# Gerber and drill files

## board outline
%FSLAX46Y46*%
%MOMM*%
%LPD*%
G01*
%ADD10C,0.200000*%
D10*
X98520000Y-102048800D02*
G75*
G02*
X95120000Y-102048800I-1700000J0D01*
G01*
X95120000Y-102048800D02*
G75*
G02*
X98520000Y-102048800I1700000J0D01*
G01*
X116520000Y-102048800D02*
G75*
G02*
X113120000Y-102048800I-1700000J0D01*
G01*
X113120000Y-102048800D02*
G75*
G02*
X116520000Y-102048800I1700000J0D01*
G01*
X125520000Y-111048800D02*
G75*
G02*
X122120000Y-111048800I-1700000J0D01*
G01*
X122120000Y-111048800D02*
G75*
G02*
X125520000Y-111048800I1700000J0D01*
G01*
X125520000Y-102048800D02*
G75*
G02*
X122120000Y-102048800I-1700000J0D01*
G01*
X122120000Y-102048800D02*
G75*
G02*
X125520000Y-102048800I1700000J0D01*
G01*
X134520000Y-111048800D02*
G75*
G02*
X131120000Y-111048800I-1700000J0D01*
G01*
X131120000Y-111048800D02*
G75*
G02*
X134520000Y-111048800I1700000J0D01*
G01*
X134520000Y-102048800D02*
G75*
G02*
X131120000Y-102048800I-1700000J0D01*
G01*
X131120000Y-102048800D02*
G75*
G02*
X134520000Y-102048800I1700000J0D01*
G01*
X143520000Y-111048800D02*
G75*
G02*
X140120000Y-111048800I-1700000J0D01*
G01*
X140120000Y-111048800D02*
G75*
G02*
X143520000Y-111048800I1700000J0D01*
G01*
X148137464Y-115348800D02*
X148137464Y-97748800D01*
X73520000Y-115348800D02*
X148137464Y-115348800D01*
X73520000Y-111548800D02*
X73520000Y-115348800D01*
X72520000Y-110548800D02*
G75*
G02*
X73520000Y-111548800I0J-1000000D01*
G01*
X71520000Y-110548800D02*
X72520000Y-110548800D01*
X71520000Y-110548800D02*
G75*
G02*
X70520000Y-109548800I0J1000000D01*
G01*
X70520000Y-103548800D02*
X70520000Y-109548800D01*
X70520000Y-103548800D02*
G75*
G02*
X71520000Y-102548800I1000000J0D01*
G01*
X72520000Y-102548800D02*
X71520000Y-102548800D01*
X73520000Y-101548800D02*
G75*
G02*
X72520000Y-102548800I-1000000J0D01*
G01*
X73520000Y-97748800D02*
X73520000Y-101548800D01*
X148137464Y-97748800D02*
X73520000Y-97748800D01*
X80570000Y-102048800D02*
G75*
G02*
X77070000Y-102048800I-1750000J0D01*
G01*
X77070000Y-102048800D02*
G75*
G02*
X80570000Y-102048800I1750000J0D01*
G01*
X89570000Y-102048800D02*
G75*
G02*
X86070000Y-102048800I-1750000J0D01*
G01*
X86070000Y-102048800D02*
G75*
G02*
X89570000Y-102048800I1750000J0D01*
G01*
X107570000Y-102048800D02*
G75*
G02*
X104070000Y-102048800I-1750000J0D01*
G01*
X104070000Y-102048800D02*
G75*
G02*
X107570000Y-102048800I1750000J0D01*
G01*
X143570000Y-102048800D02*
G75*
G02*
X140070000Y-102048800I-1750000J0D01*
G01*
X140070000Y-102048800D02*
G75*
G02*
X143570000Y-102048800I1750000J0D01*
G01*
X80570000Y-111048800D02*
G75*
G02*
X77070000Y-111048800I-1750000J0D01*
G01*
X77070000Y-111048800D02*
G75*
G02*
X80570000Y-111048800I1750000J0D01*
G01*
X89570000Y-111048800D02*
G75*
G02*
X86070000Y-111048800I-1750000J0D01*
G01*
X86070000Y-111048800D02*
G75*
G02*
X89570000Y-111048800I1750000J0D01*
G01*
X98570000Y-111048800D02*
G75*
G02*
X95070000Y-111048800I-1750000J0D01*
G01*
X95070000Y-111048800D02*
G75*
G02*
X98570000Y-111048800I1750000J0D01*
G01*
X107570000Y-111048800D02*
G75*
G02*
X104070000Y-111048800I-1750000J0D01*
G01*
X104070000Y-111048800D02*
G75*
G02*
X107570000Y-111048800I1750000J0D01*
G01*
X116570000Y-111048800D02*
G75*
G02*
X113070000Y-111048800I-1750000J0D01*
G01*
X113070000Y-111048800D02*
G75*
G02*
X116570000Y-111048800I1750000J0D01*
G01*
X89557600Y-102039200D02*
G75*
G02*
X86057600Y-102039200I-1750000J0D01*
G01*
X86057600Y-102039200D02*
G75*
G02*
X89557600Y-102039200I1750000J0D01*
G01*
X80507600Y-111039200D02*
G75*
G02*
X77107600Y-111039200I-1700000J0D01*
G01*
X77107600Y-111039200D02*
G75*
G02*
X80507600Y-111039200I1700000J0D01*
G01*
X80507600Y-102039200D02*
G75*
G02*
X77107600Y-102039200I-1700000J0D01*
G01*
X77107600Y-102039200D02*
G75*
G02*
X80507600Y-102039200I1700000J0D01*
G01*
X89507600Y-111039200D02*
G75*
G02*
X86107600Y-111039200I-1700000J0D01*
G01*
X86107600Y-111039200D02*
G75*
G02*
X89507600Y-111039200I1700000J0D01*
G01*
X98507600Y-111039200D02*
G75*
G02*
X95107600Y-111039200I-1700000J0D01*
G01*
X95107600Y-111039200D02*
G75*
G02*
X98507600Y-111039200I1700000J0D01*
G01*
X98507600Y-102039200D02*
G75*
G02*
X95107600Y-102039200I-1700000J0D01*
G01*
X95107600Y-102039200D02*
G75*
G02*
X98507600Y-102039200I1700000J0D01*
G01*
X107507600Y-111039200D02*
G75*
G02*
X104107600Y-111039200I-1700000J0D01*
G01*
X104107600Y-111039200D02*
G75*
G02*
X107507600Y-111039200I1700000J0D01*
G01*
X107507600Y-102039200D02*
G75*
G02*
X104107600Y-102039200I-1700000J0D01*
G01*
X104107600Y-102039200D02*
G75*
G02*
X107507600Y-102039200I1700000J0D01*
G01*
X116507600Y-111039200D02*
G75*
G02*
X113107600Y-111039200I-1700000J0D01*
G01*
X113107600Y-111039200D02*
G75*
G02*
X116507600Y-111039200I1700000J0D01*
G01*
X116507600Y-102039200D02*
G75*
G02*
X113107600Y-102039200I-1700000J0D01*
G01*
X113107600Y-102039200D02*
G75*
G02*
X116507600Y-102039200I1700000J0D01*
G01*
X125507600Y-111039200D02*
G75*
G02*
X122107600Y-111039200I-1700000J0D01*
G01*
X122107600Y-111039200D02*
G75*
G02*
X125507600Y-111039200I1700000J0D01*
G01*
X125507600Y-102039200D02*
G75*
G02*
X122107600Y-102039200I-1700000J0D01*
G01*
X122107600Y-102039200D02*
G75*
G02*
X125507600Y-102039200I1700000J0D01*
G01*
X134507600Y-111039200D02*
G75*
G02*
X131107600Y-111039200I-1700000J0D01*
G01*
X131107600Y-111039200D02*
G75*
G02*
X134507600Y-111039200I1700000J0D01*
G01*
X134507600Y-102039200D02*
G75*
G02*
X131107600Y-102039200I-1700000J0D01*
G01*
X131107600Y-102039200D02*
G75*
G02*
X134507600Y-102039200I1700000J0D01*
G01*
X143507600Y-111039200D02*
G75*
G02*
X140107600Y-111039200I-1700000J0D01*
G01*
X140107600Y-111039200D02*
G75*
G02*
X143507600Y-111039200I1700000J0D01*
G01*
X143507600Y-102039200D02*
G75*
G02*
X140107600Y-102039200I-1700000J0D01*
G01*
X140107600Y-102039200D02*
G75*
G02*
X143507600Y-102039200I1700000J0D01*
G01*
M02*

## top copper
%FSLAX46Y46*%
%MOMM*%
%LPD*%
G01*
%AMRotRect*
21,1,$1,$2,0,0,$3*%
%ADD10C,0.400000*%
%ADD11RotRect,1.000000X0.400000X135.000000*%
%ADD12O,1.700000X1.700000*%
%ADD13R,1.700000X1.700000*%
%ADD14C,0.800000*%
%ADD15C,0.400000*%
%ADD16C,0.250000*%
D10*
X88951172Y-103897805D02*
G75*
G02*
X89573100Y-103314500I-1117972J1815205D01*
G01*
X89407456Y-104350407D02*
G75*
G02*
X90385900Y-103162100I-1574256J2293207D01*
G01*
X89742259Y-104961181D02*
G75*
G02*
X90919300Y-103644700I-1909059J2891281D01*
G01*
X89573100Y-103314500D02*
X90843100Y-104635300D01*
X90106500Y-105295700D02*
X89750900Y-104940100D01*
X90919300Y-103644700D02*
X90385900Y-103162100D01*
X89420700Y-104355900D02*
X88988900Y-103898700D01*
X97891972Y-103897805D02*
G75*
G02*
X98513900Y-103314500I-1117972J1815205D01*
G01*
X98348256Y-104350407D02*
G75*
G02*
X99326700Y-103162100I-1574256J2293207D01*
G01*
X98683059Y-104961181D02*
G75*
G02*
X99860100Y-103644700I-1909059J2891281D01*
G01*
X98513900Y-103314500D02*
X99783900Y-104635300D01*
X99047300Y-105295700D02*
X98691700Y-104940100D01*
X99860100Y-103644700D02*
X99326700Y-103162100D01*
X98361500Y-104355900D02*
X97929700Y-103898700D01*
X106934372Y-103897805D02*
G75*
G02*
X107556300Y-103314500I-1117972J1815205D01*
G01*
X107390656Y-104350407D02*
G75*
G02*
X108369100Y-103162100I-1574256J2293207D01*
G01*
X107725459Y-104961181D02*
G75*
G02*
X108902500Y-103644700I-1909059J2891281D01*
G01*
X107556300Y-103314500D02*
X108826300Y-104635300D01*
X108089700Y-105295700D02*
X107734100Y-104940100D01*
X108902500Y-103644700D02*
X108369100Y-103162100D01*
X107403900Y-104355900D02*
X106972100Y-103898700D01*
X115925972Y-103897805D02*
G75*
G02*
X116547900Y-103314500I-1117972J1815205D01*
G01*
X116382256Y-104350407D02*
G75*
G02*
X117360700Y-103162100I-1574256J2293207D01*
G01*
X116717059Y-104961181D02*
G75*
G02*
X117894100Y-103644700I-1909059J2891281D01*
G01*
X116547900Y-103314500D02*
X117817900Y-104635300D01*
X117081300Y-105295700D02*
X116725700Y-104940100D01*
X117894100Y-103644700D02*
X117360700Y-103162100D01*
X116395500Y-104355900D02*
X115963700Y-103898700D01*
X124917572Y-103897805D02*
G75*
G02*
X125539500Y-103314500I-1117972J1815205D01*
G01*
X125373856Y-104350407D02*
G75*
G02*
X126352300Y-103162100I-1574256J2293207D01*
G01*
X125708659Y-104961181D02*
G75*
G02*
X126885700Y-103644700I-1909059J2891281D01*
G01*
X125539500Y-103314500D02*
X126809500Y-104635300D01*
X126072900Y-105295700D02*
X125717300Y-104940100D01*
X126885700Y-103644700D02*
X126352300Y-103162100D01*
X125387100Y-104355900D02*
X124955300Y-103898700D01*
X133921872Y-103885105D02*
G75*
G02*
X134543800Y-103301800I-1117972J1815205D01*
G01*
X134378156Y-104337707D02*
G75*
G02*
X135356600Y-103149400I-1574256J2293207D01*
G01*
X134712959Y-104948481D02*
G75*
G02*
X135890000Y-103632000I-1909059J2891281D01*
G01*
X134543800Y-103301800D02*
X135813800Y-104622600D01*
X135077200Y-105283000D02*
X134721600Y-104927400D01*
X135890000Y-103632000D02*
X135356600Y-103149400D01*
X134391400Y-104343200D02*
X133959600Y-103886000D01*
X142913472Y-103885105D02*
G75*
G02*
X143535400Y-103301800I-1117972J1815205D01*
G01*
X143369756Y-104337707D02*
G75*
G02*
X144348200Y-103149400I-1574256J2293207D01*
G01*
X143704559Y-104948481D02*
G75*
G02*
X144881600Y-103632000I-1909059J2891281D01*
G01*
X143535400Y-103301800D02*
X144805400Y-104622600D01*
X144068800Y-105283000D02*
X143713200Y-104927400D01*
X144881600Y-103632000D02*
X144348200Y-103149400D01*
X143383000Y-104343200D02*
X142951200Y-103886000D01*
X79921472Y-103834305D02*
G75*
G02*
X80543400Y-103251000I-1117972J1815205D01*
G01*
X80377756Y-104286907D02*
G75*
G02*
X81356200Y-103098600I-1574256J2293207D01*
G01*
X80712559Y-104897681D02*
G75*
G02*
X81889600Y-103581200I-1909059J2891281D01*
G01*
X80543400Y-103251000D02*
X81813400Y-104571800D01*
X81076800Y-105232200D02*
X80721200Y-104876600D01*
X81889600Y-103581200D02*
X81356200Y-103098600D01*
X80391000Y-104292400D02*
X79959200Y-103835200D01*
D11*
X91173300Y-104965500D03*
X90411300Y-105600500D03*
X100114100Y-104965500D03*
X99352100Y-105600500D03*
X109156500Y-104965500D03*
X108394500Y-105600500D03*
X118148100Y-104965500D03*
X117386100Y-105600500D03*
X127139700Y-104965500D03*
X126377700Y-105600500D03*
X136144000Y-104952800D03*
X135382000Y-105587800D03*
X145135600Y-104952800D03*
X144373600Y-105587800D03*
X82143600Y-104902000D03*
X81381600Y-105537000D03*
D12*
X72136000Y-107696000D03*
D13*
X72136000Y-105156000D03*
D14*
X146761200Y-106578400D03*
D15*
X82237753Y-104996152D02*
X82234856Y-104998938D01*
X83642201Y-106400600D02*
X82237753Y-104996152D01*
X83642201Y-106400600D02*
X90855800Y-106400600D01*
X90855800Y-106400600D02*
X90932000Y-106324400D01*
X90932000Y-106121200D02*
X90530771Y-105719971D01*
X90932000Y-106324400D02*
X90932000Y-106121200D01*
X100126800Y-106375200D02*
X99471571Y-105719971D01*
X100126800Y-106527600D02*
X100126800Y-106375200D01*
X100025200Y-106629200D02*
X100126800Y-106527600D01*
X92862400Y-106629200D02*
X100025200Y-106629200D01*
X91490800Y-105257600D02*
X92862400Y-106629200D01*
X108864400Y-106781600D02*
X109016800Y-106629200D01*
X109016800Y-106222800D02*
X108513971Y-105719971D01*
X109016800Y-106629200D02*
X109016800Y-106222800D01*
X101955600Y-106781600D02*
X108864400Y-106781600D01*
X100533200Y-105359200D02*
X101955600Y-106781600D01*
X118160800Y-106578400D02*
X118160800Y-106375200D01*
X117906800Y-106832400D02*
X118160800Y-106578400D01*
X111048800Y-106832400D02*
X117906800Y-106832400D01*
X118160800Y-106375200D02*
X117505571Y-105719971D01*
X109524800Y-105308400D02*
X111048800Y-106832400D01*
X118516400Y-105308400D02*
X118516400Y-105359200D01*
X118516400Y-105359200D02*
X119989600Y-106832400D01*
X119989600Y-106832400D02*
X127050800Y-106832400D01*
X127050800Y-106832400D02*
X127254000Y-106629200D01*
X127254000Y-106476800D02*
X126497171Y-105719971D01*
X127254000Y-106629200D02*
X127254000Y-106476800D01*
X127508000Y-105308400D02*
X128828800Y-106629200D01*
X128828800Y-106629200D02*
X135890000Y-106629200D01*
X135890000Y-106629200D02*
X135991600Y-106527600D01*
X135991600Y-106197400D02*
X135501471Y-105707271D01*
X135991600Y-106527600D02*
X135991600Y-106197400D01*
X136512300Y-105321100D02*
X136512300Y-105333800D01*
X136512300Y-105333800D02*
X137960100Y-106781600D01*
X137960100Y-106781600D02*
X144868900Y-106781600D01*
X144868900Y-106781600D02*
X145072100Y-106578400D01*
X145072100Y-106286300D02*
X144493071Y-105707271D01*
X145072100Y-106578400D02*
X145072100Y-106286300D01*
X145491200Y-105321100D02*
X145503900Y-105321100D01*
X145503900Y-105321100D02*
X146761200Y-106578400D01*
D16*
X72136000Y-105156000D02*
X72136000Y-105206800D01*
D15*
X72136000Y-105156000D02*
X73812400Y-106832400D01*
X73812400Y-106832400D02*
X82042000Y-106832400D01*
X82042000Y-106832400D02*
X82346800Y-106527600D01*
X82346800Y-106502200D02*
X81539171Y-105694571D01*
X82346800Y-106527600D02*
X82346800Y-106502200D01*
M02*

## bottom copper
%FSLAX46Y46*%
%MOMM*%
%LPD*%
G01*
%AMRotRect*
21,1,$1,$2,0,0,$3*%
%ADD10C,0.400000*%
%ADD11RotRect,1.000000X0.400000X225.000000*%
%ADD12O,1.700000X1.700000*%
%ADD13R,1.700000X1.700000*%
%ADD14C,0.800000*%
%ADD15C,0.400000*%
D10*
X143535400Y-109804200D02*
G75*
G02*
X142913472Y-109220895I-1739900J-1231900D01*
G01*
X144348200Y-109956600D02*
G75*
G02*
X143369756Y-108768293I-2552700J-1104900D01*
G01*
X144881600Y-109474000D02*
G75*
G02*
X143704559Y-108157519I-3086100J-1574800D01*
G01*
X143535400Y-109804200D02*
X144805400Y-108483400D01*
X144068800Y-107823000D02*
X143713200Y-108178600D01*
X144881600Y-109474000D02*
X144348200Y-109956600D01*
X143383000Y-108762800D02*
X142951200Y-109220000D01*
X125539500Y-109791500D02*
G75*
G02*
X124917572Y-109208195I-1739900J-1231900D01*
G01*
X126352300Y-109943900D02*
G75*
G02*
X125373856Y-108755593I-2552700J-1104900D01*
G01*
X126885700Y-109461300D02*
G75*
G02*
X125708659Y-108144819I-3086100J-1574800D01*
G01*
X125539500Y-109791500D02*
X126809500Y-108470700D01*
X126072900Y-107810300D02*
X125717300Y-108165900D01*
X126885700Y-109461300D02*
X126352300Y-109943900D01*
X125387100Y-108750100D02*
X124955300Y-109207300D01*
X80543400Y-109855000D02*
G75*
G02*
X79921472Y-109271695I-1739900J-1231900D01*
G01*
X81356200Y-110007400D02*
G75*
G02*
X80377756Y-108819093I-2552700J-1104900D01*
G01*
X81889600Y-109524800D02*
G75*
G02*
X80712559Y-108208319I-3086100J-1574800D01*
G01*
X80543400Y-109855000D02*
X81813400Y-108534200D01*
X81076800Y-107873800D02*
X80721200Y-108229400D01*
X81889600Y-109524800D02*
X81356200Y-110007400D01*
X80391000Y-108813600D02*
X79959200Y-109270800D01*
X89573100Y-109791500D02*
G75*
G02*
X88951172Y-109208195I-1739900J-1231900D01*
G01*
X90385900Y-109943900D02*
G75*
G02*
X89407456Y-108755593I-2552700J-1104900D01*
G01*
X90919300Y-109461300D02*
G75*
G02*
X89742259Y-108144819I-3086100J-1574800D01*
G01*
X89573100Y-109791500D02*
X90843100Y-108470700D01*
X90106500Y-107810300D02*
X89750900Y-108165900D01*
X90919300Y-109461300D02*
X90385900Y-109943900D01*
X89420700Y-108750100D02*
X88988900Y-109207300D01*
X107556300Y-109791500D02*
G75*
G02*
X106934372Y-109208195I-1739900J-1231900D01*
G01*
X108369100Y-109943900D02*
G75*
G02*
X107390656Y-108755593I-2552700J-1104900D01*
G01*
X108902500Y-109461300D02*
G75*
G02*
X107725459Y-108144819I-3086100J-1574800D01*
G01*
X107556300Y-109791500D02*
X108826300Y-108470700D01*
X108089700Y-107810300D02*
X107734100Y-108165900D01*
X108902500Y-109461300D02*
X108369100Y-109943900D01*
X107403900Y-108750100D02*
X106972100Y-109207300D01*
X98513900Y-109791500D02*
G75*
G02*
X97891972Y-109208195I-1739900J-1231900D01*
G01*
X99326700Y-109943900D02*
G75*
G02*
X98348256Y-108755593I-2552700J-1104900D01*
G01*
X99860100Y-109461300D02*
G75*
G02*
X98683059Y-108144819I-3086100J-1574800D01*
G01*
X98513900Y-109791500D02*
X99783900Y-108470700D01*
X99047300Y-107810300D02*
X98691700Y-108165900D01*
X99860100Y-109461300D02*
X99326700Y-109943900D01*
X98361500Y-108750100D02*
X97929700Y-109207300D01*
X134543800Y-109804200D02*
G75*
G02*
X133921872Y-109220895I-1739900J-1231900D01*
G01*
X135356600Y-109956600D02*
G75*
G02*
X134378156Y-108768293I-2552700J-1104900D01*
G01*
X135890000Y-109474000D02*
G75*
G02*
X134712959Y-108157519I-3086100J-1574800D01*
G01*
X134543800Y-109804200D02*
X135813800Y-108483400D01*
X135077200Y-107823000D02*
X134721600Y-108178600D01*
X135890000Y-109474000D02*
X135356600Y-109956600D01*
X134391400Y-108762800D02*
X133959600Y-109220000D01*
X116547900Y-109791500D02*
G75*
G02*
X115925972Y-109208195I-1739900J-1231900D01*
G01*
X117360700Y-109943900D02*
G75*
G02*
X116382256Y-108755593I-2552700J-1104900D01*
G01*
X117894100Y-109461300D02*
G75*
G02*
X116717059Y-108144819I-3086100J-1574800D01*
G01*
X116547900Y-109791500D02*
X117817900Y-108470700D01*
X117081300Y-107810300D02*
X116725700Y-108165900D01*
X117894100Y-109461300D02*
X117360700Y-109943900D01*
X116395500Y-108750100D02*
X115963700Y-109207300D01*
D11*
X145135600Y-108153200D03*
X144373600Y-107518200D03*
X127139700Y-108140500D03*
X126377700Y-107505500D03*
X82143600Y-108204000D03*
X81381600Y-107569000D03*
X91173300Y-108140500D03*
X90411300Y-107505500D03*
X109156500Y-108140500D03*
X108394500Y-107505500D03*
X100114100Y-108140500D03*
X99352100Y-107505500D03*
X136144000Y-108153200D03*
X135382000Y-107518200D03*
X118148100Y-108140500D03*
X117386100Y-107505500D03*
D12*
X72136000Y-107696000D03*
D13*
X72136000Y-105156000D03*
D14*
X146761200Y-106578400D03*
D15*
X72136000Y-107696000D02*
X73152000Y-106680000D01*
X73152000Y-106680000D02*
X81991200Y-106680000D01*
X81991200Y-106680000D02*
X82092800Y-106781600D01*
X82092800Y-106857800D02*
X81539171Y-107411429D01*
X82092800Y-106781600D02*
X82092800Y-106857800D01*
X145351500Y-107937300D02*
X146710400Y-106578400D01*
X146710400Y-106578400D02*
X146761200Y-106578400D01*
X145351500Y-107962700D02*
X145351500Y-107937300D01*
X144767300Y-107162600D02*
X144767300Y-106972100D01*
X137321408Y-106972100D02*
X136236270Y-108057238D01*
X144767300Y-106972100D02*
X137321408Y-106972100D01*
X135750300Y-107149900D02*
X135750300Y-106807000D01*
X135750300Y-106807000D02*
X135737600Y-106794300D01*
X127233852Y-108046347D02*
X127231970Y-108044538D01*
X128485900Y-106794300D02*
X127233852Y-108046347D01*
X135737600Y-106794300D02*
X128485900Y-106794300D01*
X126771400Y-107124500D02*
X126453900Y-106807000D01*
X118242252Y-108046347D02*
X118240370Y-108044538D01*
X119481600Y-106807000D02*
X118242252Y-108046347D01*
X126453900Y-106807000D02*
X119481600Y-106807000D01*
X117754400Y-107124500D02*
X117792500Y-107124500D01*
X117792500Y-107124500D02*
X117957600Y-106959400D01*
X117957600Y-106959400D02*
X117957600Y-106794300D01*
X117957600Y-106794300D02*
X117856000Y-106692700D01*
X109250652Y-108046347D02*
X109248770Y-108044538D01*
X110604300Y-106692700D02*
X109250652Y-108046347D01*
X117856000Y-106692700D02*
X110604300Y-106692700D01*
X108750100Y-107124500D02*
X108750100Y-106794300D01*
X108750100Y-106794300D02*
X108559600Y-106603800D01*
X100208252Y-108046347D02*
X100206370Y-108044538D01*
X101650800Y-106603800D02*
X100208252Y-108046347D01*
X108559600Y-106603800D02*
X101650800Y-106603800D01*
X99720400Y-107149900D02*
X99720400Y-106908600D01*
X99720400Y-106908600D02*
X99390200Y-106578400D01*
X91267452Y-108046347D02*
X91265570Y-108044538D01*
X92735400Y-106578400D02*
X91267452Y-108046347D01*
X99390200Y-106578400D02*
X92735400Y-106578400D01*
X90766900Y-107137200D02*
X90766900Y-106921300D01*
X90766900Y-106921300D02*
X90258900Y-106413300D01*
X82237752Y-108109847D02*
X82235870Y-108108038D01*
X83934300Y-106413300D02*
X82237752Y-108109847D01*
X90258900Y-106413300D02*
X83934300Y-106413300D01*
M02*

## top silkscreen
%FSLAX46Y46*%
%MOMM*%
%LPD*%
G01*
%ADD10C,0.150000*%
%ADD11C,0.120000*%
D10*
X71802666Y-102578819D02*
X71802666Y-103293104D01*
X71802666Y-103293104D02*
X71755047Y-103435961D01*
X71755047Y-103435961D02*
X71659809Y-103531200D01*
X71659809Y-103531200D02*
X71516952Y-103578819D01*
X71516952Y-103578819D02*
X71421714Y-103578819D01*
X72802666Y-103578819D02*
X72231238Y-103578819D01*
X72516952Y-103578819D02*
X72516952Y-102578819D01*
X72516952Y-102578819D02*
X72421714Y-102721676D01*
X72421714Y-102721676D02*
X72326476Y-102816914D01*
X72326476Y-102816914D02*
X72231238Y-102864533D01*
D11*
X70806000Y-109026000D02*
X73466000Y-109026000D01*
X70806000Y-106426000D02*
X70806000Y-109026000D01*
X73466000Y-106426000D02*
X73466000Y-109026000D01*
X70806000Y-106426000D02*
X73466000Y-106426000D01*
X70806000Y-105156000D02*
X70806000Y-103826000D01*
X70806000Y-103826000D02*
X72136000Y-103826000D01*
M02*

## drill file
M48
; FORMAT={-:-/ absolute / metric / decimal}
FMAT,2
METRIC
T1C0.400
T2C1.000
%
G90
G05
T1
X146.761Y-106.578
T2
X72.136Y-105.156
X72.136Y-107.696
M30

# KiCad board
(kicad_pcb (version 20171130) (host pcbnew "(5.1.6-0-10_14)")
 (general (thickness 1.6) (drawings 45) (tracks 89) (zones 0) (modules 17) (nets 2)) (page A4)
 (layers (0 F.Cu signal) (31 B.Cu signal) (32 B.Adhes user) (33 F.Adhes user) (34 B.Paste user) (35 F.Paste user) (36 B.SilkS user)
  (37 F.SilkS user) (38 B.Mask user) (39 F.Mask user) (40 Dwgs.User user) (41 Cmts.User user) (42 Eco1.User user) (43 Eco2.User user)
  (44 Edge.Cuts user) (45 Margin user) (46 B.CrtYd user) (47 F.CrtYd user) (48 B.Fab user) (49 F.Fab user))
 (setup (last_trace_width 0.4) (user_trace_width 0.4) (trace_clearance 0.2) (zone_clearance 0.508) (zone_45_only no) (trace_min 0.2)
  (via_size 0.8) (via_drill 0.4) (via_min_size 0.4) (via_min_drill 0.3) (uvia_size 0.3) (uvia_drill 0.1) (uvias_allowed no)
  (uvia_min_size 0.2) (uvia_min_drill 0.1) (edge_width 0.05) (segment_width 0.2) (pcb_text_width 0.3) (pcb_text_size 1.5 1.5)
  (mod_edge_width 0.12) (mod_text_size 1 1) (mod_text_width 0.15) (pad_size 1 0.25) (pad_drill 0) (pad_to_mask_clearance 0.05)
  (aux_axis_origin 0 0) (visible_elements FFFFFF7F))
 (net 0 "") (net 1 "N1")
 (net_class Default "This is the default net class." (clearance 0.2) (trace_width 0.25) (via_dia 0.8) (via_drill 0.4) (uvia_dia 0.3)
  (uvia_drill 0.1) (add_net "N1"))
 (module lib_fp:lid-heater (layer F.Cu) (at 88.1761 108.2167)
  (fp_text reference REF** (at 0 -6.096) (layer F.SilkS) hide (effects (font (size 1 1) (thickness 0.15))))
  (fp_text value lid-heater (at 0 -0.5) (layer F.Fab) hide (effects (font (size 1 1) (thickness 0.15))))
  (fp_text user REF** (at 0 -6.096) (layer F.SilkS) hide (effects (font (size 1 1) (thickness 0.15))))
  (fp_arc (start -0.3429 -6.1341) (end 1.397 -4.9022) (angle -336.9282282) (layer F.Cu) (width 0.4))
  (fp_arc (start -0.3429 -6.1595) (end 2.2098 -5.0546) (angle -327.8737649) (layer F.Cu) (width 0.4))
  (fp_arc (start -0.3429 -6.1468) (end 2.7432 -4.572) (angle -330.4707161) (layer F.Cu) (width 0.4))
  (fp_line (start 1.397 -4.9022) (end 2.667 -3.5814) (layer F.Cu) (width 0.4))
  (fp_line (start 1.9304 -2.921) (end 1.5748 -3.2766) (layer F.Cu) (width 0.4))
  (fp_line (start 2.7432 -4.572) (end 2.2098 -5.0546) (layer F.Cu) (width 0.4))
  (fp_line (start 1.2446 -3.8608) (end 0.8128 -4.318) (layer F.Cu) (width 0.4))
  (pad 1 smd rect (at 2.9972 -3.2512 135) (size 1 0.4) (layers F.Cu F.Paste))
  (pad 1 smd rect (at 2.2352 -2.6162 135) (size 1 0.4) (layers F.Cu F.Paste)))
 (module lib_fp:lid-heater (layer F.Cu) (at 97.1169 108.2167)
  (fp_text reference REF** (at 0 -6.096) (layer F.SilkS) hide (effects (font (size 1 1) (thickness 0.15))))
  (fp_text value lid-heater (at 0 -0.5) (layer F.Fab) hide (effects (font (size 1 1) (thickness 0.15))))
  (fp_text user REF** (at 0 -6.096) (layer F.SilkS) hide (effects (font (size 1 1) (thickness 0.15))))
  (fp_arc (start -0.3429 -6.1341) (end 1.397 -4.9022) (angle -336.9282282) (layer F.Cu) (width 0.4))
  (fp_arc (start -0.3429 -6.1595) (end 2.2098 -5.0546) (angle -327.8737649) (layer F.Cu) (width 0.4))
  (fp_arc (start -0.3429 -6.1468) (end 2.7432 -4.572) (angle -330.4707161) (layer F.Cu) (width 0.4))
  (fp_line (start 1.397 -4.9022) (end 2.667 -3.5814) (layer F.Cu) (width 0.4))
  (fp_line (start 1.9304 -2.921) (end 1.5748 -3.2766) (layer F.Cu) (width 0.4))
  (fp_line (start 2.7432 -4.572) (end 2.2098 -5.0546) (layer F.Cu) (width 0.4))
  (fp_line (start 1.2446 -3.8608) (end 0.8128 -4.318) (layer F.Cu) (width 0.4))
  (pad 1 smd rect (at 2.9972 -3.2512 135) (size 1 0.4) (layers F.Cu F.Paste))
  (pad 1 smd rect (at 2.2352 -2.6162 135) (size 1 0.4) (layers F.Cu F.Paste)))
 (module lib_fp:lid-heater (layer F.Cu) (at 106.1593 108.2167)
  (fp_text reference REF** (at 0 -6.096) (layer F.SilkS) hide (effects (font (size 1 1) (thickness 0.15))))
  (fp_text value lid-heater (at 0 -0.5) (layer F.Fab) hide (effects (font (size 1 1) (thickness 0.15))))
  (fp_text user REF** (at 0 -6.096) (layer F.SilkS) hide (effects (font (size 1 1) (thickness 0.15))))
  (fp_arc (start -0.3429 -6.1341) (end 1.397 -4.9022) (angle -336.9282282) (layer F.Cu) (width 0.4))
  (fp_arc (start -0.3429 -6.1595) (end 2.2098 -5.0546) (angle -327.8737649) (layer F.Cu) (width 0.4))
  (fp_arc (start -0.3429 -6.1468) (end 2.7432 -4.572) (angle -330.4707161) (layer F.Cu) (width 0.4))
  (fp_line (start 1.397 -4.9022) (end 2.667 -3.5814) (layer F.Cu) (width 0.4))
  (fp_line (start 1.9304 -2.921) (end 1.5748 -3.2766) (layer F.Cu) (width 0.4))
  (fp_line (start 2.7432 -4.572) (end 2.2098 -5.0546) (layer F.Cu) (width 0.4))
  (fp_line (start 1.2446 -3.8608) (end 0.8128 -4.318) (layer F.Cu) (width 0.4))
  (pad 1 smd rect (at 2.9972 -3.2512 135) (size 1 0.4) (layers F.Cu F.Paste))
  (pad 1 smd rect (at 2.2352 -2.6162 135) (size 1 0.4) (layers F.Cu F.Paste)))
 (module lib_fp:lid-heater (layer F.Cu) (at 115.1509 108.2167)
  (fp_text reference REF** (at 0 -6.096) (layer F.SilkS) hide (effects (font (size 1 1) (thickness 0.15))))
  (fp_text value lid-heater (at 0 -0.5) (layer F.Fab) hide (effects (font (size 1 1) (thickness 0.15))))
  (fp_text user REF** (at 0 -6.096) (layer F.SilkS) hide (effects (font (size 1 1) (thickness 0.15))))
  (fp_arc (start -0.3429 -6.1341) (end 1.397 -4.9022) (angle -336.9282282) (layer F.Cu) (width 0.4))
  (fp_arc (start -0.3429 -6.1595) (end 2.2098 -5.0546) (angle -327.8737649) (layer F.Cu) (width 0.4))
  (fp_arc (start -0.3429 -6.1468) (end 2.7432 -4.572) (angle -330.4707161) (layer F.Cu) (width 0.4))
  (fp_line (start 1.397 -4.9022) (end 2.667 -3.5814) (layer F.Cu) (width 0.4))
  (fp_line (start 1.9304 -2.921) (end 1.5748 -3.2766) (layer F.Cu) (width 0.4))
  (fp_line (start 2.7432 -4.572) (end 2.2098 -5.0546) (layer F.Cu) (width 0.4))
  (fp_line (start 1.2446 -3.8608) (end 0.8128 -4.318) (layer F.Cu) (width 0.4))
  (pad 1 smd rect (at 2.9972 -3.2512 135) (size 1 0.4) (layers F.Cu F.Paste))
  (pad 1 smd rect (at 2.2352 -2.6162 135) (size 1 0.4) (layers F.Cu F.Paste)))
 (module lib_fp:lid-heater (layer F.Cu) (at 124.1425 108.2167)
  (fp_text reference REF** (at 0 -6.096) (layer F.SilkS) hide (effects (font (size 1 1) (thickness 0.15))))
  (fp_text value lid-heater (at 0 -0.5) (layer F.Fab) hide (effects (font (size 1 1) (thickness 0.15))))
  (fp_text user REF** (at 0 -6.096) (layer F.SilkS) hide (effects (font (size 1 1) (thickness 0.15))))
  (fp_arc (start -0.3429 -6.1341) (end 1.397 -4.9022) (angle -336.9282282) (layer F.Cu) (width 0.4))
  (fp_arc (start -0.3429 -6.1595) (end 2.2098 -5.0546) (angle -327.8737649) (layer F.Cu) (width 0.4))
  (fp_arc (start -0.3429 -6.1468) (end 2.7432 -4.572) (angle -330.4707161) (layer F.Cu) (width 0.4))
  (fp_line (start 1.397 -4.9022) (end 2.667 -3.5814) (layer F.Cu) (width 0.4))
  (fp_line (start 1.9304 -2.921) (end 1.5748 -3.2766) (layer F.Cu) (width 0.4))
  (fp_line (start 2.7432 -4.572) (end 2.2098 -5.0546) (layer F.Cu) (width 0.4))
  (fp_line (start 1.2446 -3.8608) (end 0.8128 -4.318) (layer F.Cu) (width 0.4))
  (pad 1 smd rect (at 2.9972 -3.2512 135) (size 1 0.4) (layers F.Cu F.Paste))
  (pad 1 smd rect (at 2.2352 -2.6162 135) (size 1 0.4) (layers F.Cu F.Paste)))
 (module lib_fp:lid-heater (layer F.Cu) (at 133.1468 108.204)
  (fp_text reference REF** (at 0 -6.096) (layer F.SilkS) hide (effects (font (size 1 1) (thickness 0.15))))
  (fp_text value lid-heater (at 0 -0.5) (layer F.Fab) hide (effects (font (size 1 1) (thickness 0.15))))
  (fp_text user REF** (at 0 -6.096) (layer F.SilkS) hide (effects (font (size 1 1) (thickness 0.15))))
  (fp_arc (start -0.3429 -6.1341) (end 1.397 -4.9022) (angle -336.9282282) (layer F.Cu) (width 0.4))
  (fp_arc (start -0.3429 -6.1595) (end 2.2098 -5.0546) (angle -327.8737649) (layer F.Cu) (width 0.4))
  (fp_arc (start -0.3429 -6.1468) (end 2.7432 -4.572) (angle -330.4707161) (layer F.Cu) (width 0.4))
  (fp_line (start 1.397 -4.9022) (end 2.667 -3.5814) (layer F.Cu) (width 0.4))
  (fp_line (start 1.9304 -2.921) (end 1.5748 -3.2766) (layer F.Cu) (width 0.4))
  (fp_line (start 2.7432 -4.572) (end 2.2098 -5.0546) (layer F.Cu) (width 0.4))
  (fp_line (start 1.2446 -3.8608) (end 0.8128 -4.318) (layer F.Cu) (width 0.4))
  (pad 1 smd rect (at 2.9972 -3.2512 135) (size 1 0.4) (layers F.Cu F.Paste))
  (pad 1 smd rect (at 2.2352 -2.6162 135) (size 1 0.4) (layers F.Cu F.Paste)))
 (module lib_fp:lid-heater (layer F.Cu) (at 142.1384 108.204)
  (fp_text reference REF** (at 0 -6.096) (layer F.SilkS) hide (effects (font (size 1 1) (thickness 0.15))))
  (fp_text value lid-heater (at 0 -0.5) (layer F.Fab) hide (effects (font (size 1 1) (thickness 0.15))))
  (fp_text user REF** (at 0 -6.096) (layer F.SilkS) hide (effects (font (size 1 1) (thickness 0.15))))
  (fp_arc (start -0.3429 -6.1341) (end 1.397 -4.9022) (angle -336.9282282) (layer F.Cu) (width 0.4))
  (fp_arc (start -0.3429 -6.1595) (end 2.2098 -5.0546) (angle -327.8737649) (layer F.Cu) (width 0.4))
  (fp_arc (start -0.3429 -6.1468) (end 2.7432 -4.572) (angle -330.4707161) (layer F.Cu) (width 0.4))
  (fp_line (start 1.397 -4.9022) (end 2.667 -3.5814) (layer F.Cu) (width 0.4))
  (fp_line (start 1.9304 -2.921) (end 1.5748 -3.2766) (layer F.Cu) (width 0.4))
  (fp_line (start 2.7432 -4.572) (end 2.2098 -5.0546) (layer F.Cu) (width 0.4))
  (fp_line (start 1.2446 -3.8608) (end 0.8128 -4.318) (layer F.Cu) (width 0.4))
  (pad 1 smd rect (at 2.9972 -3.2512 135) (size 1 0.4) (layers F.Cu F.Paste))
  (pad 1 smd rect (at 2.2352 -2.6162 135) (size 1 0.4) (layers F.Cu F.Paste)))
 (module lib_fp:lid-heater (layer B.Cu) (at 142.1384 104.902)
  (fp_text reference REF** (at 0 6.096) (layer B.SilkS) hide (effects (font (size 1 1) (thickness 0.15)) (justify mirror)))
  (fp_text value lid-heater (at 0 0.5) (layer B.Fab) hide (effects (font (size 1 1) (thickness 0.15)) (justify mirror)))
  (fp_arc (start -0.3429 6.1341) (end 1.397 4.9022) (angle 336.9282282) (layer B.Cu) (width 0.4))
  (fp_arc (start -0.3429 6.1595) (end 2.2098 5.0546) (angle 327.8737649) (layer B.Cu) (width 0.4))
  (fp_arc (start -0.3429 6.1468) (end 2.7432 4.572) (angle 330.4707161) (layer B.Cu) (width 0.4))
  (fp_line (start 1.397 4.9022) (end 2.667 3.5814) (layer B.Cu) (width 0.4))
  (fp_line (start 1.9304 2.921) (end 1.5748 3.2766) (layer B.Cu) (width 0.4))
  (fp_line (start 2.7432 4.572) (end 2.2098 5.0546) (layer B.Cu) (width 0.4))
  (fp_line (start 1.2446 3.8608) (end 0.8128 4.318) (layer B.Cu) (width 0.4))
  (pad 1 smd rect (at 2.9972 3.2512 225) (size 1 0.4) (layers B.Cu B.Paste))
  (pad 1 smd rect (at 2.2352 2.6162 225) (size 1 0.4) (layers B.Cu B.Paste)))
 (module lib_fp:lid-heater (layer B.Cu) (at 124.1425 104.8893)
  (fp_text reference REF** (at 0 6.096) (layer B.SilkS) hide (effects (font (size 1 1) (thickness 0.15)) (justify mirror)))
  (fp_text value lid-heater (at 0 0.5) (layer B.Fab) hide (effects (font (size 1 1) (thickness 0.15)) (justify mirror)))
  (fp_arc (start -0.3429 6.1341) (end 1.397 4.9022) (angle 336.9282282) (layer B.Cu) (width 0.4))
  (fp_arc (start -0.3429 6.1595) (end 2.2098 5.0546) (angle 327.8737649) (layer B.Cu) (width 0.4))
  (fp_arc (start -0.3429 6.1468) (end 2.7432 4.572) (angle 330.4707161) (layer B.Cu) (width 0.4))
  (fp_line (start 1.397 4.9022) (end 2.667 3.5814) (layer B.Cu) (width 0.4))
  (fp_line (start 1.9304 2.921) (end 1.5748 3.2766) (layer B.Cu) (width 0.4))
  (fp_line (start 2.7432 4.572) (end 2.2098 5.0546) (layer B.Cu) (width 0.4))
  (fp_line (start 1.2446 3.8608) (end 0.8128 4.318) (layer B.Cu) (width 0.4))
  (pad 1 smd rect (at 2.9972 3.2512 225) (size 1 0.4) (layers B.Cu B.Paste))
  (pad 1 smd rect (at 2.2352 2.6162 225) (size 1 0.4) (layers B.Cu B.Paste)))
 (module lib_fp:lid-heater (layer B.Cu) (at 79.1464 104.9528)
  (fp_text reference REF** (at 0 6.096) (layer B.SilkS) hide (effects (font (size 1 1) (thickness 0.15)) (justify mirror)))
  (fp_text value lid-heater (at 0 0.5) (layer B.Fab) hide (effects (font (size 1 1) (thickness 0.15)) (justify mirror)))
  (fp_arc (start -0.3429 6.1341) (end 1.397 4.9022) (angle 336.9282282) (layer B.Cu) (width 0.4))
  (fp_arc (start -0.3429 6.1595) (end 2.2098 5.0546) (angle 327.8737649) (layer B.Cu) (width 0.4))
  (fp_arc (start -0.3429 6.1468) (end 2.7432 4.572) (angle 330.4707161) (layer B.Cu) (width 0.4))
  (fp_line (start 1.397 4.9022) (end 2.667 3.5814) (layer B.Cu) (width 0.4))
  (fp_line (start 1.9304 2.921) (end 1.5748 3.2766) (layer B.Cu) (width 0.4))
  (fp_line (start 2.7432 4.572) (end 2.2098 5.0546) (layer B.Cu) (width 0.4))
  (fp_line (start 1.2446 3.8608) (end 0.8128 4.318) (layer B.Cu) (width 0.4))
  (pad 1 smd rect (at 2.9972 3.2512 225) (size 1 0.4) (layers B.Cu B.Paste))
  (pad 1 smd rect (at 2.2352 2.6162 225) (size 1 0.4) (layers B.Cu B.Paste)))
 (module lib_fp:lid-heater (layer B.Cu) (at 88.1761 104.8893)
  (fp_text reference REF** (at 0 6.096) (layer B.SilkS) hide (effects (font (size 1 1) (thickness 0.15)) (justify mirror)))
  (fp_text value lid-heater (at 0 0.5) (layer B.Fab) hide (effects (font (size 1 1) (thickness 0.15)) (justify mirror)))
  (fp_arc (start -0.3429 6.1341) (end 1.397 4.9022) (angle 336.9282282) (layer B.Cu) (width 0.4))
  (fp_arc (start -0.3429 6.1595) (end 2.2098 5.0546) (angle 327.8737649) (layer B.Cu) (width 0.4))
  (fp_arc (start -0.3429 6.1468) (end 2.7432 4.572) (angle 330.4707161) (layer B.Cu) (width 0.4))
  (fp_line (start 1.397 4.9022) (end 2.667 3.5814) (layer B.Cu) (width 0.4))
  (fp_line (start 1.9304 2.921) (end 1.5748 3.2766) (layer B.Cu) (width 0.4))
  (fp_line (start 2.7432 4.572) (end 2.2098 5.0546) (layer B.Cu) (width 0.4))
  (fp_line (start 1.2446 3.8608) (end 0.8128 4.318) (layer B.Cu) (width 0.4))
  (pad 1 smd rect (at 2.9972 3.2512 225) (size 1 0.4) (layers B.Cu B.Paste))
  (pad 1 smd rect (at 2.2352 2.6162 225) (size 1 0.4) (layers B.Cu B.Paste)))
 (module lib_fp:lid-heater (layer B.Cu) (at 106.1593 104.8893)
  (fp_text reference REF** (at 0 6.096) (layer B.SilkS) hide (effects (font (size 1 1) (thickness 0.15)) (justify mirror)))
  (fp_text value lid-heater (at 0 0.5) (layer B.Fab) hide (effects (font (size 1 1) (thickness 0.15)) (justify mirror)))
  (fp_arc (start -0.3429 6.1341) (end 1.397 4.9022) (angle 336.9282282) (layer B.Cu) (width 0.4))
  (fp_arc (start -0.3429 6.1595) (end 2.2098 5.0546) (angle 327.8737649) (layer B.Cu) (width 0.4))
  (fp_arc (start -0.3429 6.1468) (end 2.7432 4.572) (angle 330.4707161) (layer B.Cu) (width 0.4))
  (fp_line (start 1.397 4.9022) (end 2.667 3.5814) (layer B.Cu) (width 0.4))
  (fp_line (start 1.9304 2.921) (end 1.5748 3.2766) (layer B.Cu) (width 0.4))
  (fp_line (start 2.7432 4.572) (end 2.2098 5.0546) (layer B.Cu) (width 0.4))
  (fp_line (start 1.2446 3.8608) (end 0.8128 4.318) (layer B.Cu) (width 0.4))
  (pad 1 smd rect (at 2.9972 3.2512 225) (size 1 0.4) (layers B.Cu B.Paste))
  (pad 1 smd rect (at 2.2352 2.6162 225) (size 1 0.4) (layers B.Cu B.Paste)))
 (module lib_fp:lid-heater (layer B.Cu) (at 97.1169 104.8893)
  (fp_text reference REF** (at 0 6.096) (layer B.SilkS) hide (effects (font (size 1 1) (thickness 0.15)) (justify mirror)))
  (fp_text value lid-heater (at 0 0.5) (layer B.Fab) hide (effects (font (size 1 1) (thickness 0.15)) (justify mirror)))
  (fp_arc (start -0.3429 6.1341) (end 1.397 4.9022) (angle 336.9282282) (layer B.Cu) (width 0.4))
  (fp_arc (start -0.3429 6.1595) (end 2.2098 5.0546) (angle 327.8737649) (layer B.Cu) (width 0.4))
  (fp_arc (start -0.3429 6.1468) (end 2.7432 4.572) (angle 330.4707161) (layer B.Cu) (width 0.4))
  (fp_line (start 1.397 4.9022) (end 2.667 3.5814) (layer B.Cu) (width 0.4))
  (fp_line (start 1.9304 2.921) (end 1.5748 3.2766) (layer B.Cu) (width 0.4))
  (fp_line (start 2.7432 4.572) (end 2.2098 5.0546) (layer B.Cu) (width 0.4))
  (fp_line (start 1.2446 3.8608) (end 0.8128 4.318) (layer B.Cu) (width 0.4))
  (pad 1 smd rect (at 2.9972 3.2512 225) (size 1 0.4) (layers B.Cu B.Paste))
  (pad 1 smd rect (at 2.2352 2.6162 225) (size 1 0.4) (layers B.Cu B.Paste)))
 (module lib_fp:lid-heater (layer B.Cu) (at 133.1468 104.902)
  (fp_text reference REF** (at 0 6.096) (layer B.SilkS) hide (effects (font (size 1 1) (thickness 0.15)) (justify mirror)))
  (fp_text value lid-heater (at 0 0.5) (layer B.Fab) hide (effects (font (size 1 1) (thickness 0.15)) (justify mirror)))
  (fp_arc (start -0.3429 6.1341) (end 1.397 4.9022) (angle 336.9282282) (layer B.Cu) (width 0.4))
  (fp_arc (start -0.3429 6.1595) (end 2.2098 5.0546) (angle 327.8737649) (layer B.Cu) (width 0.4))
  (fp_arc (start -0.3429 6.1468) (end 2.7432 4.572) (angle 330.4707161) (layer B.Cu) (width 0.4))
  (fp_line (start 1.397 4.9022) (end 2.667 3.5814) (layer B.Cu) (width 0.4))
  (fp_line (start 1.9304 2.921) (end 1.5748 3.2766) (layer B.Cu) (width 0.4))
  (fp_line (start 2.7432 4.572) (end 2.2098 5.0546) (layer B.Cu) (width 0.4))
  (fp_line (start 1.2446 3.8608) (end 0.8128 4.318) (layer B.Cu) (width 0.4))
  (pad 1 smd rect (at 2.9972 3.2512 225) (size 1 0.4) (layers B.Cu B.Paste))
  (pad 1 smd rect (at 2.2352 2.6162 225) (size 1 0.4) (layers B.Cu B.Paste)))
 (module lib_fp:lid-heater (layer B.Cu) (at 115.1509 104.8893)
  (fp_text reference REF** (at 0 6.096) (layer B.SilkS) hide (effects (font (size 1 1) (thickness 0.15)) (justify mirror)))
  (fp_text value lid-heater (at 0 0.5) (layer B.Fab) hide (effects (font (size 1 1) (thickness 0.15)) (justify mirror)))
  (fp_arc (start -0.3429 6.1341) (end 1.397 4.9022) (angle 336.9282282) (layer B.Cu) (width 0.4))
  (fp_arc (start -0.3429 6.1595) (end 2.2098 5.0546) (angle 327.8737649) (layer B.Cu) (width 0.4))
  (fp_arc (start -0.3429 6.1468) (end 2.7432 4.572) (angle 330.4707161) (layer B.Cu) (width 0.4))
  (fp_line (start 1.397 4.9022) (end 2.667 3.5814) (layer B.Cu) (width 0.4))
  (fp_line (start 1.9304 2.921) (end 1.5748 3.2766) (layer B.Cu) (width 0.4))
  (fp_line (start 2.7432 4.572) (end 2.2098 5.0546) (layer B.Cu) (width 0.4))
  (fp_line (start 1.2446 3.8608) (end 0.8128 4.318) (layer B.Cu) (width 0.4))
  (pad 1 smd rect (at 2.9972 3.2512 225) (size 1 0.4) (layers B.Cu B.Paste))
  (pad 1 smd rect (at 2.2352 2.6162 225) (size 1 0.4) (layers B.Cu B.Paste)))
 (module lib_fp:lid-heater (layer F.Cu) (at 79.1464 108.1532)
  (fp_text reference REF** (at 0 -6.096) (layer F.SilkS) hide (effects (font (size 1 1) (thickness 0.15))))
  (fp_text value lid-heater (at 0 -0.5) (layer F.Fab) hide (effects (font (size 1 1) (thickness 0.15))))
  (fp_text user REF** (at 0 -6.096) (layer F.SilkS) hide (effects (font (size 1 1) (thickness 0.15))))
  (fp_arc (start -0.3429 -6.1341) (end 1.397 -4.9022) (angle -336.9282282) (layer F.Cu) (width 0.4))
  (fp_arc (start -0.3429 -6.1595) (end 2.2098 -5.0546) (angle -327.8737649) (layer F.Cu) (width 0.4))
  (fp_arc (start -0.3429 -6.1468) (end 2.7432 -4.572) (angle -330.4707161) (layer F.Cu) (width 0.4))
  (fp_line (start 1.397 -4.9022) (end 2.667 -3.5814) (layer F.Cu) (width 0.4))
  (fp_line (start 1.9304 -2.921) (end 1.5748 -3.2766) (layer F.Cu) (width 0.4))
  (fp_line (start 2.7432 -4.572) (end 2.2098 -5.0546) (layer F.Cu) (width 0.4))
  (fp_line (start 1.2446 -3.8608) (end 0.8128 -4.318) (layer F.Cu) (width 0.4))
  (pad 1 smd rect (at 2.9972 -3.2512 135) (size 1 0.4) (layers F.Cu F.Paste))
  (pad 1 smd rect (at 2.2352 -2.6162 135) (size 1 0.4) (layers F.Cu F.Paste)))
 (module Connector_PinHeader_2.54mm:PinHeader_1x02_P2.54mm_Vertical (layer F.Cu) (at 72.136 105.156)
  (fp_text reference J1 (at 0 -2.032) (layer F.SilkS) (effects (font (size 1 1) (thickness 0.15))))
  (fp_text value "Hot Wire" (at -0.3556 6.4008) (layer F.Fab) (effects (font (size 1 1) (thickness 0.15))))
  (fp_line (start -1.33 3.87) (end 1.33 3.87) (layer F.SilkS) (width 0.12))
  (fp_line (start -1.33 1.27) (end -1.33 3.87) (layer F.SilkS) (width 0.12))
  (fp_line (start 1.33 1.27) (end 1.33 3.87) (layer F.SilkS) (width 0.12))
  (fp_line (start -1.33 1.27) (end 1.33 1.27) (layer F.SilkS) (width 0.12))
  (fp_line (start -1.33 0) (end -1.33 -1.33) (layer F.SilkS) (width 0.12))
  (fp_line (start -1.33 -1.33) (end 0 -1.33) (layer F.SilkS) (width 0.12))
  (pad 2 thru_hole oval (at 0 2.54) (size 1.7 1.7) (drill 1) (layers *.Cu *.Mask))
  (pad 1 thru_hole rect (at 0 0) (size 1.7 1.7) (drill 1) (layers *.Cu *.Mask) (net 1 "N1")))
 (gr_circle (center 96.82 102.0488) (end 96.82 103.7488) (layer Edge.Cuts) (width 0.2))
 (gr_circle (center 114.82 102.0488) (end 114.82 103.7488) (layer Edge.Cuts) (width 0.2))
 (gr_circle (center 123.82 111.0488) (end 123.82 112.7488) (layer Edge.Cuts) (width 0.2))
 (gr_circle (center 123.82 102.0488) (end 123.82 103.7488) (layer Edge.Cuts) (width 0.2))
 (gr_circle (center 132.82 111.0488) (end 132.82 112.7488) (layer Edge.Cuts) (width 0.2))
 (gr_circle (center 132.82 102.0488) (end 132.82 103.7488) (layer Edge.Cuts) (width 0.2))
 (gr_circle (center 141.82 111.0488) (end 141.82 112.7488) (layer Edge.Cuts) (width 0.2))
 (gr_line (start 148.137464 115.3488) (end 148.137464 97.7488) (layer Edge.Cuts) (width 0.2))
 (gr_line (start 73.52 115.3488) (end 148.137464 115.3488) (layer Edge.Cuts) (width 0.2))
 (gr_line (start 73.52 111.5488) (end 73.52 115.3488) (layer Edge.Cuts) (width 0.2))
 (gr_arc (start 72.52 111.5488) (end 73.52 111.5488) (angle -90) (layer Edge.Cuts) (width 0.2))
 (gr_line (start 71.52 110.5488) (end 72.52 110.5488) (layer Edge.Cuts) (width 0.2))
 (gr_arc (start 71.52 109.5488) (end 70.52 109.5488) (angle -90) (layer Edge.Cuts) (width 0.2))
 (gr_line (start 70.52 103.5488) (end 70.52 109.5488) (layer Edge.Cuts) (width 0.2))
 (gr_arc (start 71.52 103.5488) (end 71.52 102.5488) (angle -90) (layer Edge.Cuts) (width 0.2))
 (gr_line (start 72.52 102.5488) (end 71.52 102.5488) (layer Edge.Cuts) (width 0.2))
 (gr_arc (start 72.52 101.5488) (end 72.52 102.5488) (angle -90) (layer Edge.Cuts) (width 0.2))
 (gr_line (start 73.52 97.7488) (end 73.52 101.5488) (layer Edge.Cuts) (width 0.2))
 (gr_line (start 148.137464 97.7488) (end 73.52 97.7488) (layer Edge.Cuts) (width 0.2))
 (gr_circle (center 78.82 102.0488) (end 78.82 103.7988) (layer Edge.Cuts) (width 0.2))
 (gr_circle (center 87.82 102.0488) (end 87.82 103.7988) (layer Edge.Cuts) (width 0.2))
 (gr_circle (center 105.82 102.0488) (end 105.82 103.7988) (layer Edge.Cuts) (width 0.2))
 (gr_circle (center 141.82 102.0488) (end 141.82 103.7988) (layer Edge.Cuts) (width 0.2))
 (gr_circle (center 78.82 111.0488) (end 78.82 112.7988) (layer Edge.Cuts) (width 0.2))
 (gr_circle (center 87.82 111.0488) (end 87.82 112.7988) (layer Edge.Cuts) (width 0.2))
 (gr_circle (center 96.82 111.0488) (end 96.82 112.7988) (layer Edge.Cuts) (width 0.2))
 (gr_circle (center 105.82 111.0488) (end 105.82 112.7988) (layer Edge.Cuts) (width 0.2))
 (gr_circle (center 114.82 111.0488) (end 114.82 112.7988) (layer Edge.Cuts) (width 0.2))
 (gr_circle (center 87.8076 102.0392) (end 87.8076 103.7892) (layer Edge.Cuts) (width 0.2))
 (gr_circle (center 78.8076 111.0392) (end 78.8076 112.7392) (layer Edge.Cuts) (width 0.2))
 (gr_circle (center 78.8076 102.0392) (end 78.8076 103.7392) (layer Edge.Cuts) (width 0.2))
 (gr_circle (center 87.8076 111.0392) (end 87.8076 112.7392) (layer Edge.Cuts) (width 0.2))
 (gr_circle (center 96.8076 111.0392) (end 96.8076 112.7392) (layer Edge.Cuts) (width 0.2))
 (gr_circle (center 96.8076 102.0392) (end 96.8076 103.7392) (layer Edge.Cuts) (width 0.2))
 (gr_circle (center 105.8076 111.0392) (end 105.8076 112.7392) (layer Edge.Cuts) (width 0.2))
 (gr_circle (center 105.8076 102.0392) (end 105.8076 103.7392) (layer Edge.Cuts) (width 0.2))
 (gr_circle (center 114.8076 111.0392) (end 114.8076 112.7392) (layer Edge.Cuts) (width 0.2))
 (gr_circle (center 114.8076 102.0392) (end 114.8076 103.7392) (layer Edge.Cuts) (width 0.2))
 (gr_circle (center 123.8076 111.0392) (end 123.8076 112.7392) (layer Edge.Cuts) (width 0.2))
 (gr_circle (center 123.8076 102.0392) (end 123.8076 103.7392) (layer Edge.Cuts) (width 0.2))
 (gr_circle (center 132.8076 111.0392) (end 132.8076 112.7392) (layer Edge.Cuts) (width 0.2))
 (gr_circle (center 132.8076 102.0392) (end 132.8076 103.7392) (layer Edge.Cuts) (width 0.2))
 (gr_circle (center 141.8076 111.0392) (end 141.8076 112.7392) (layer Edge.Cuts) (width 0.2))
 (gr_circle (center 141.8076 102.0392) (end 141.8076 103.7392) (layer Edge.Cuts) (width 0.2))
 (segment (start 72.136 107.696) (end 73.152 106.68) (width 0.4) (layer B.Cu) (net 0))
 (segment (start 73.152 106.68) (end 81.9912 106.68) (width 0.4) (layer B.Cu) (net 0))
 (segment (start 81.9912 106.68) (end 82.0928 106.7816) (width 0.4) (layer B.Cu) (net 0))
 (segment (start 82.0928 106.8578) (end 81.539171 107.411429) (width 0.4) (layer B.Cu) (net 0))
 (segment (start 82.0928 106.7816) (end 82.0928 106.8578) (width 0.4) (layer B.Cu) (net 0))
 (segment (start 82.237753 104.996152) (end 82.234856 104.998938) (width 0.4) (layer F.Cu) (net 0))
 (segment (start 83.642201 106.4006) (end 82.237753 104.996152) (width 0.4) (layer F.Cu) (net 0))
 (segment (start 83.642201 106.4006) (end 90.8558 106.4006) (width 0.4) (layer F.Cu) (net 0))
 (segment (start 90.8558 106.4006) (end 90.932 106.3244) (width 0.4) (layer F.Cu) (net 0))
 (segment (start 90.932 106.1212) (end 90.530771 105.719971) (width 0.4) (layer F.Cu) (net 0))
 (segment (start 90.932 106.3244) (end 90.932 106.1212) (width 0.4) (layer F.Cu) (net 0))
 (segment (start 100.1268 106.3752) (end 99.471571 105.719971) (width 0.4) (layer F.Cu) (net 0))
 (segment (start 100.1268 106.5276) (end 100.1268 106.3752) (width 0.4) (layer F.Cu) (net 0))
 (segment (start 100.0252 106.6292) (end 100.1268 106.5276) (width 0.4) (layer F.Cu) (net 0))
 (segment (start 92.8624 106.6292) (end 100.0252 106.6292) (width 0.4) (layer F.Cu) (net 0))
 (segment (start 91.4908 105.2576) (end 92.8624 106.6292) (width 0.4) (layer F.Cu) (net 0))
 (segment (start 108.8644 106.7816) (end 109.0168 106.6292) (width 0.4) (layer F.Cu) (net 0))
 (segment (start 109.0168 106.2228) (end 108.513971 105.719971) (width 0.4) (layer F.Cu) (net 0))
 (segment (start 109.0168 106.6292) (end 109.0168 106.2228) (width 0.4) (layer F.Cu) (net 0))
 (segment (start 101.9556 106.7816) (end 108.8644 106.7816) (width 0.4) (layer F.Cu) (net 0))
 (segment (start 100.5332 105.3592) (end 101.9556 106.7816) (width 0.4) (layer F.Cu) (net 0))
 (segment (start 118.1608 106.5784) (end 118.1608 106.3752) (width 0.4) (layer F.Cu) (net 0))
 (segment (start 117.9068 106.8324) (end 118.1608 106.5784) (width 0.4) (layer F.Cu) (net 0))
 (segment (start 111.0488 106.8324) (end 117.9068 106.8324) (width 0.4) (layer F.Cu) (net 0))
 (segment (start 118.1608 106.3752) (end 117.505571 105.719971) (width 0.4) (layer F.Cu) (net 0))
 (segment (start 109.5248 105.3084) (end 111.0488 106.8324) (width 0.4) (layer F.Cu) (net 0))
 (segment (start 118.5164 105.3084) (end 118.5164 105.3592) (width 0.4) (layer F.Cu) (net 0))
 (segment (start 118.5164 105.3592) (end 119.9896 106.8324) (width 0.4) (layer F.Cu) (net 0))
 (segment (start 119.9896 106.8324) (end 127.0508 106.8324) (width 0.4) (layer F.Cu) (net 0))
 (segment (start 127.0508 106.8324) (end 127.254 106.6292) (width 0.4) (layer F.Cu) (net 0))
 (segment (start 127.254 106.4768) (end 126.497171 105.719971) (width 0.4) (layer F.Cu) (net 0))
 (segment (start 127.254 106.6292) (end 127.254 106.4768) (width 0.4) (layer F.Cu) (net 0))
 (segment (start 127.508 105.3084) (end 128.8288 106.6292) (width 0.4) (layer F.Cu) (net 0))
 (segment (start 128.8288 106.6292) (end 135.89 106.6292) (width 0.4) (layer F.Cu) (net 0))
 (segment (start 135.89 106.6292) (end 135.9916 106.5276) (width 0.4) (layer F.Cu) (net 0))
 (segment (start 135.9916 106.1974) (end 135.501471 105.707271) (width 0.4) (layer F.Cu) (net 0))
 (segment (start 135.9916 106.5276) (end 135.9916 106.1974) (width 0.4) (layer F.Cu) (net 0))
 (segment (start 136.5123 105.3211) (end 136.5123 105.3338) (width 0.4) (layer F.Cu) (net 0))
 (segment (start 136.5123 105.3338) (end 137.9601 106.7816) (width 0.4) (layer F.Cu) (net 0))
 (segment (start 137.9601 106.7816) (end 144.8689 106.7816) (width 0.4) (layer F.Cu) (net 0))
 (segment (start 144.8689 106.7816) (end 145.0721 106.5784) (width 0.4) (layer F.Cu) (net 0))
 (segment (start 145.0721 106.2863) (end 144.493071 105.707271) (width 0.4) (layer F.Cu) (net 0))
 (segment (start 145.0721 106.5784) (end 145.0721 106.2863) (width 0.4) (layer F.Cu) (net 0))
 (segment (start 145.4912 105.3211) (end 145.5039 105.3211) (width 0.4) (layer F.Cu) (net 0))
 (segment (start 145.5039 105.3211) (end 146.7612 106.5784) (width 0.4) (layer F.Cu) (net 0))
 (via (at 146.7612 106.5784) (size 0.8) (drill 0.4) (layers F.Cu B.Cu) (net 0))
 (segment (start 145.3515 107.9373) (end 146.7104 106.5784) (width 0.4) (layer B.Cu) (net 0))
 (segment (start 146.7104 106.5784) (end 146.7612 106.5784) (width 0.4) (layer B.Cu) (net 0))
 (segment (start 145.3515 107.9627) (end 145.3515 107.9373) (width 0.4) (layer B.Cu) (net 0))
 (segment (start 144.7673 107.1626) (end 144.7673 106.9721) (width 0.4) (layer B.Cu) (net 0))
 (segment (start 137.321408 106.9721) (end 136.23627 108.057238) (width 0.4) (layer B.Cu) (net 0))
 (segment (start 144.7673 106.9721) (end 137.321408 106.9721) (width 0.4) (layer B.Cu) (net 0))
 (segment (start 135.7503 107.1499) (end 135.7503 106.807) (width 0.4) (layer B.Cu) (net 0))
 (segment (start 135.7503 106.807) (end 135.7376 106.7943) (width 0.4) (layer B.Cu) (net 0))
 (segment (start 127.233852 108.046347) (end 127.23197 108.044538) (width 0.4) (layer B.Cu) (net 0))
 (segment (start 128.4859 106.7943) (end 127.233852 108.046347) (width 0.4) (layer B.Cu) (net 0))
 (segment (start 135.7376 106.7943) (end 128.4859 106.7943) (width 0.4) (layer B.Cu) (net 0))
 (segment (start 126.7714 107.1245) (end 126.4539 106.807) (width 0.4) (layer B.Cu) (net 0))
 (segment (start 118.242252 108.046347) (end 118.24037 108.044538) (width 0.4) (layer B.Cu) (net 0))
 (segment (start 119.4816 106.807) (end 118.242252 108.046347) (width 0.4) (layer B.Cu) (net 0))
 (segment (start 126.4539 106.807) (end 119.4816 106.807) (width 0.4) (layer B.Cu) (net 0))
 (segment (start 117.7544 107.1245) (end 117.7925 107.1245) (width 0.4) (layer B.Cu) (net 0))
 (segment (start 117.7925 107.1245) (end 117.9576 106.9594) (width 0.4) (layer B.Cu) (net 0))
 (segment (start 117.9576 106.9594) (end 117.9576 106.7943) (width 0.4) (layer B.Cu) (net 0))
 (segment (start 117.9576 106.7943) (end 117.856 106.6927) (width 0.4) (layer B.Cu) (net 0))
 (segment (start 109.250652 108.046347) (end 109.24877 108.044538) (width 0.4) (layer B.Cu) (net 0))
 (segment (start 110.6043 106.6927) (end 109.250652 108.046347) (width 0.4) (layer B.Cu) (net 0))
 (segment (start 117.856 106.6927) (end 110.6043 106.6927) (width 0.4) (layer B.Cu) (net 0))
 (segment (start 108.7501 107.1245) (end 108.7501 106.7943) (width 0.4) (layer B.Cu) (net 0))
 (segment (start 108.7501 106.7943) (end 108.5596 106.6038) (width 0.4) (layer B.Cu) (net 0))
 (segment (start 100.208252 108.046347) (end 100.20637 108.044538) (width 0.4) (layer B.Cu) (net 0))
 (segment (start 101.6508 106.6038) (end 100.208252 108.046347) (width 0.4) (layer B.Cu) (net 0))
 (segment (start 108.5596 106.6038) (end 101.6508 106.6038) (width 0.4) (layer B.Cu) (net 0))
 (segment (start 99.7204 107.1499) (end 99.7204 106.9086) (width 0.4) (layer B.Cu) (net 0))
 (segment (start 99.7204 106.9086) (end 99.3902 106.5784) (width 0.4) (layer B.Cu) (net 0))
 (segment (start 91.267452 108.046347) (end 91.26557 108.044538) (width 0.4) (layer B.Cu) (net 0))
 (segment (start 92.7354 106.5784) (end 91.267452 108.046347) (width 0.4) (layer B.Cu) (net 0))
 (segment (start 99.3902 106.5784) (end 92.7354 106.5784) (width 0.4) (layer B.Cu) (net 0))
 (segment (start 90.7669 107.1372) (end 90.7669 106.9213) (width 0.4) (layer B.Cu) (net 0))
 (segment (start 90.7669 106.9213) (end 90.2589 106.4133) (width 0.4) (layer B.Cu) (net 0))
 (segment (start 82.237752 108.109847) (end 82.23587 108.108038) (width 0.4) (layer B.Cu) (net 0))
 (segment (start 83.9343 106.4133) (end 82.237752 108.109847) (width 0.4) (layer B.Cu) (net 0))
 (segment (start 90.2589 106.4133) (end 83.9343 106.4133) (width 0.4) (layer B.Cu) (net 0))
 (segment (start 72.136 105.156) (end 72.136 105.2068) (width 0.25) (layer F.Cu) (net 1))
 (segment (start 72.136 105.156) (end 73.8124 106.8324) (width 0.4) (layer F.Cu) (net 1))
 (segment (start 73.8124 106.8324) (end 82.042 106.8324) (width 0.4) (layer F.Cu) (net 1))
 (segment (start 82.042 106.8324) (end 82.3468 106.5276) (width 0.4) (layer F.Cu) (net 1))
 (segment (start 82.3468 106.5022) (end 81.539171 105.694571) (width 0.4) (layer F.Cu) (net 1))
 (segment (start 82.3468 106.5276) (end 82.3468 106.5022) (width 0.4) (layer F.Cu) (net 1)))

